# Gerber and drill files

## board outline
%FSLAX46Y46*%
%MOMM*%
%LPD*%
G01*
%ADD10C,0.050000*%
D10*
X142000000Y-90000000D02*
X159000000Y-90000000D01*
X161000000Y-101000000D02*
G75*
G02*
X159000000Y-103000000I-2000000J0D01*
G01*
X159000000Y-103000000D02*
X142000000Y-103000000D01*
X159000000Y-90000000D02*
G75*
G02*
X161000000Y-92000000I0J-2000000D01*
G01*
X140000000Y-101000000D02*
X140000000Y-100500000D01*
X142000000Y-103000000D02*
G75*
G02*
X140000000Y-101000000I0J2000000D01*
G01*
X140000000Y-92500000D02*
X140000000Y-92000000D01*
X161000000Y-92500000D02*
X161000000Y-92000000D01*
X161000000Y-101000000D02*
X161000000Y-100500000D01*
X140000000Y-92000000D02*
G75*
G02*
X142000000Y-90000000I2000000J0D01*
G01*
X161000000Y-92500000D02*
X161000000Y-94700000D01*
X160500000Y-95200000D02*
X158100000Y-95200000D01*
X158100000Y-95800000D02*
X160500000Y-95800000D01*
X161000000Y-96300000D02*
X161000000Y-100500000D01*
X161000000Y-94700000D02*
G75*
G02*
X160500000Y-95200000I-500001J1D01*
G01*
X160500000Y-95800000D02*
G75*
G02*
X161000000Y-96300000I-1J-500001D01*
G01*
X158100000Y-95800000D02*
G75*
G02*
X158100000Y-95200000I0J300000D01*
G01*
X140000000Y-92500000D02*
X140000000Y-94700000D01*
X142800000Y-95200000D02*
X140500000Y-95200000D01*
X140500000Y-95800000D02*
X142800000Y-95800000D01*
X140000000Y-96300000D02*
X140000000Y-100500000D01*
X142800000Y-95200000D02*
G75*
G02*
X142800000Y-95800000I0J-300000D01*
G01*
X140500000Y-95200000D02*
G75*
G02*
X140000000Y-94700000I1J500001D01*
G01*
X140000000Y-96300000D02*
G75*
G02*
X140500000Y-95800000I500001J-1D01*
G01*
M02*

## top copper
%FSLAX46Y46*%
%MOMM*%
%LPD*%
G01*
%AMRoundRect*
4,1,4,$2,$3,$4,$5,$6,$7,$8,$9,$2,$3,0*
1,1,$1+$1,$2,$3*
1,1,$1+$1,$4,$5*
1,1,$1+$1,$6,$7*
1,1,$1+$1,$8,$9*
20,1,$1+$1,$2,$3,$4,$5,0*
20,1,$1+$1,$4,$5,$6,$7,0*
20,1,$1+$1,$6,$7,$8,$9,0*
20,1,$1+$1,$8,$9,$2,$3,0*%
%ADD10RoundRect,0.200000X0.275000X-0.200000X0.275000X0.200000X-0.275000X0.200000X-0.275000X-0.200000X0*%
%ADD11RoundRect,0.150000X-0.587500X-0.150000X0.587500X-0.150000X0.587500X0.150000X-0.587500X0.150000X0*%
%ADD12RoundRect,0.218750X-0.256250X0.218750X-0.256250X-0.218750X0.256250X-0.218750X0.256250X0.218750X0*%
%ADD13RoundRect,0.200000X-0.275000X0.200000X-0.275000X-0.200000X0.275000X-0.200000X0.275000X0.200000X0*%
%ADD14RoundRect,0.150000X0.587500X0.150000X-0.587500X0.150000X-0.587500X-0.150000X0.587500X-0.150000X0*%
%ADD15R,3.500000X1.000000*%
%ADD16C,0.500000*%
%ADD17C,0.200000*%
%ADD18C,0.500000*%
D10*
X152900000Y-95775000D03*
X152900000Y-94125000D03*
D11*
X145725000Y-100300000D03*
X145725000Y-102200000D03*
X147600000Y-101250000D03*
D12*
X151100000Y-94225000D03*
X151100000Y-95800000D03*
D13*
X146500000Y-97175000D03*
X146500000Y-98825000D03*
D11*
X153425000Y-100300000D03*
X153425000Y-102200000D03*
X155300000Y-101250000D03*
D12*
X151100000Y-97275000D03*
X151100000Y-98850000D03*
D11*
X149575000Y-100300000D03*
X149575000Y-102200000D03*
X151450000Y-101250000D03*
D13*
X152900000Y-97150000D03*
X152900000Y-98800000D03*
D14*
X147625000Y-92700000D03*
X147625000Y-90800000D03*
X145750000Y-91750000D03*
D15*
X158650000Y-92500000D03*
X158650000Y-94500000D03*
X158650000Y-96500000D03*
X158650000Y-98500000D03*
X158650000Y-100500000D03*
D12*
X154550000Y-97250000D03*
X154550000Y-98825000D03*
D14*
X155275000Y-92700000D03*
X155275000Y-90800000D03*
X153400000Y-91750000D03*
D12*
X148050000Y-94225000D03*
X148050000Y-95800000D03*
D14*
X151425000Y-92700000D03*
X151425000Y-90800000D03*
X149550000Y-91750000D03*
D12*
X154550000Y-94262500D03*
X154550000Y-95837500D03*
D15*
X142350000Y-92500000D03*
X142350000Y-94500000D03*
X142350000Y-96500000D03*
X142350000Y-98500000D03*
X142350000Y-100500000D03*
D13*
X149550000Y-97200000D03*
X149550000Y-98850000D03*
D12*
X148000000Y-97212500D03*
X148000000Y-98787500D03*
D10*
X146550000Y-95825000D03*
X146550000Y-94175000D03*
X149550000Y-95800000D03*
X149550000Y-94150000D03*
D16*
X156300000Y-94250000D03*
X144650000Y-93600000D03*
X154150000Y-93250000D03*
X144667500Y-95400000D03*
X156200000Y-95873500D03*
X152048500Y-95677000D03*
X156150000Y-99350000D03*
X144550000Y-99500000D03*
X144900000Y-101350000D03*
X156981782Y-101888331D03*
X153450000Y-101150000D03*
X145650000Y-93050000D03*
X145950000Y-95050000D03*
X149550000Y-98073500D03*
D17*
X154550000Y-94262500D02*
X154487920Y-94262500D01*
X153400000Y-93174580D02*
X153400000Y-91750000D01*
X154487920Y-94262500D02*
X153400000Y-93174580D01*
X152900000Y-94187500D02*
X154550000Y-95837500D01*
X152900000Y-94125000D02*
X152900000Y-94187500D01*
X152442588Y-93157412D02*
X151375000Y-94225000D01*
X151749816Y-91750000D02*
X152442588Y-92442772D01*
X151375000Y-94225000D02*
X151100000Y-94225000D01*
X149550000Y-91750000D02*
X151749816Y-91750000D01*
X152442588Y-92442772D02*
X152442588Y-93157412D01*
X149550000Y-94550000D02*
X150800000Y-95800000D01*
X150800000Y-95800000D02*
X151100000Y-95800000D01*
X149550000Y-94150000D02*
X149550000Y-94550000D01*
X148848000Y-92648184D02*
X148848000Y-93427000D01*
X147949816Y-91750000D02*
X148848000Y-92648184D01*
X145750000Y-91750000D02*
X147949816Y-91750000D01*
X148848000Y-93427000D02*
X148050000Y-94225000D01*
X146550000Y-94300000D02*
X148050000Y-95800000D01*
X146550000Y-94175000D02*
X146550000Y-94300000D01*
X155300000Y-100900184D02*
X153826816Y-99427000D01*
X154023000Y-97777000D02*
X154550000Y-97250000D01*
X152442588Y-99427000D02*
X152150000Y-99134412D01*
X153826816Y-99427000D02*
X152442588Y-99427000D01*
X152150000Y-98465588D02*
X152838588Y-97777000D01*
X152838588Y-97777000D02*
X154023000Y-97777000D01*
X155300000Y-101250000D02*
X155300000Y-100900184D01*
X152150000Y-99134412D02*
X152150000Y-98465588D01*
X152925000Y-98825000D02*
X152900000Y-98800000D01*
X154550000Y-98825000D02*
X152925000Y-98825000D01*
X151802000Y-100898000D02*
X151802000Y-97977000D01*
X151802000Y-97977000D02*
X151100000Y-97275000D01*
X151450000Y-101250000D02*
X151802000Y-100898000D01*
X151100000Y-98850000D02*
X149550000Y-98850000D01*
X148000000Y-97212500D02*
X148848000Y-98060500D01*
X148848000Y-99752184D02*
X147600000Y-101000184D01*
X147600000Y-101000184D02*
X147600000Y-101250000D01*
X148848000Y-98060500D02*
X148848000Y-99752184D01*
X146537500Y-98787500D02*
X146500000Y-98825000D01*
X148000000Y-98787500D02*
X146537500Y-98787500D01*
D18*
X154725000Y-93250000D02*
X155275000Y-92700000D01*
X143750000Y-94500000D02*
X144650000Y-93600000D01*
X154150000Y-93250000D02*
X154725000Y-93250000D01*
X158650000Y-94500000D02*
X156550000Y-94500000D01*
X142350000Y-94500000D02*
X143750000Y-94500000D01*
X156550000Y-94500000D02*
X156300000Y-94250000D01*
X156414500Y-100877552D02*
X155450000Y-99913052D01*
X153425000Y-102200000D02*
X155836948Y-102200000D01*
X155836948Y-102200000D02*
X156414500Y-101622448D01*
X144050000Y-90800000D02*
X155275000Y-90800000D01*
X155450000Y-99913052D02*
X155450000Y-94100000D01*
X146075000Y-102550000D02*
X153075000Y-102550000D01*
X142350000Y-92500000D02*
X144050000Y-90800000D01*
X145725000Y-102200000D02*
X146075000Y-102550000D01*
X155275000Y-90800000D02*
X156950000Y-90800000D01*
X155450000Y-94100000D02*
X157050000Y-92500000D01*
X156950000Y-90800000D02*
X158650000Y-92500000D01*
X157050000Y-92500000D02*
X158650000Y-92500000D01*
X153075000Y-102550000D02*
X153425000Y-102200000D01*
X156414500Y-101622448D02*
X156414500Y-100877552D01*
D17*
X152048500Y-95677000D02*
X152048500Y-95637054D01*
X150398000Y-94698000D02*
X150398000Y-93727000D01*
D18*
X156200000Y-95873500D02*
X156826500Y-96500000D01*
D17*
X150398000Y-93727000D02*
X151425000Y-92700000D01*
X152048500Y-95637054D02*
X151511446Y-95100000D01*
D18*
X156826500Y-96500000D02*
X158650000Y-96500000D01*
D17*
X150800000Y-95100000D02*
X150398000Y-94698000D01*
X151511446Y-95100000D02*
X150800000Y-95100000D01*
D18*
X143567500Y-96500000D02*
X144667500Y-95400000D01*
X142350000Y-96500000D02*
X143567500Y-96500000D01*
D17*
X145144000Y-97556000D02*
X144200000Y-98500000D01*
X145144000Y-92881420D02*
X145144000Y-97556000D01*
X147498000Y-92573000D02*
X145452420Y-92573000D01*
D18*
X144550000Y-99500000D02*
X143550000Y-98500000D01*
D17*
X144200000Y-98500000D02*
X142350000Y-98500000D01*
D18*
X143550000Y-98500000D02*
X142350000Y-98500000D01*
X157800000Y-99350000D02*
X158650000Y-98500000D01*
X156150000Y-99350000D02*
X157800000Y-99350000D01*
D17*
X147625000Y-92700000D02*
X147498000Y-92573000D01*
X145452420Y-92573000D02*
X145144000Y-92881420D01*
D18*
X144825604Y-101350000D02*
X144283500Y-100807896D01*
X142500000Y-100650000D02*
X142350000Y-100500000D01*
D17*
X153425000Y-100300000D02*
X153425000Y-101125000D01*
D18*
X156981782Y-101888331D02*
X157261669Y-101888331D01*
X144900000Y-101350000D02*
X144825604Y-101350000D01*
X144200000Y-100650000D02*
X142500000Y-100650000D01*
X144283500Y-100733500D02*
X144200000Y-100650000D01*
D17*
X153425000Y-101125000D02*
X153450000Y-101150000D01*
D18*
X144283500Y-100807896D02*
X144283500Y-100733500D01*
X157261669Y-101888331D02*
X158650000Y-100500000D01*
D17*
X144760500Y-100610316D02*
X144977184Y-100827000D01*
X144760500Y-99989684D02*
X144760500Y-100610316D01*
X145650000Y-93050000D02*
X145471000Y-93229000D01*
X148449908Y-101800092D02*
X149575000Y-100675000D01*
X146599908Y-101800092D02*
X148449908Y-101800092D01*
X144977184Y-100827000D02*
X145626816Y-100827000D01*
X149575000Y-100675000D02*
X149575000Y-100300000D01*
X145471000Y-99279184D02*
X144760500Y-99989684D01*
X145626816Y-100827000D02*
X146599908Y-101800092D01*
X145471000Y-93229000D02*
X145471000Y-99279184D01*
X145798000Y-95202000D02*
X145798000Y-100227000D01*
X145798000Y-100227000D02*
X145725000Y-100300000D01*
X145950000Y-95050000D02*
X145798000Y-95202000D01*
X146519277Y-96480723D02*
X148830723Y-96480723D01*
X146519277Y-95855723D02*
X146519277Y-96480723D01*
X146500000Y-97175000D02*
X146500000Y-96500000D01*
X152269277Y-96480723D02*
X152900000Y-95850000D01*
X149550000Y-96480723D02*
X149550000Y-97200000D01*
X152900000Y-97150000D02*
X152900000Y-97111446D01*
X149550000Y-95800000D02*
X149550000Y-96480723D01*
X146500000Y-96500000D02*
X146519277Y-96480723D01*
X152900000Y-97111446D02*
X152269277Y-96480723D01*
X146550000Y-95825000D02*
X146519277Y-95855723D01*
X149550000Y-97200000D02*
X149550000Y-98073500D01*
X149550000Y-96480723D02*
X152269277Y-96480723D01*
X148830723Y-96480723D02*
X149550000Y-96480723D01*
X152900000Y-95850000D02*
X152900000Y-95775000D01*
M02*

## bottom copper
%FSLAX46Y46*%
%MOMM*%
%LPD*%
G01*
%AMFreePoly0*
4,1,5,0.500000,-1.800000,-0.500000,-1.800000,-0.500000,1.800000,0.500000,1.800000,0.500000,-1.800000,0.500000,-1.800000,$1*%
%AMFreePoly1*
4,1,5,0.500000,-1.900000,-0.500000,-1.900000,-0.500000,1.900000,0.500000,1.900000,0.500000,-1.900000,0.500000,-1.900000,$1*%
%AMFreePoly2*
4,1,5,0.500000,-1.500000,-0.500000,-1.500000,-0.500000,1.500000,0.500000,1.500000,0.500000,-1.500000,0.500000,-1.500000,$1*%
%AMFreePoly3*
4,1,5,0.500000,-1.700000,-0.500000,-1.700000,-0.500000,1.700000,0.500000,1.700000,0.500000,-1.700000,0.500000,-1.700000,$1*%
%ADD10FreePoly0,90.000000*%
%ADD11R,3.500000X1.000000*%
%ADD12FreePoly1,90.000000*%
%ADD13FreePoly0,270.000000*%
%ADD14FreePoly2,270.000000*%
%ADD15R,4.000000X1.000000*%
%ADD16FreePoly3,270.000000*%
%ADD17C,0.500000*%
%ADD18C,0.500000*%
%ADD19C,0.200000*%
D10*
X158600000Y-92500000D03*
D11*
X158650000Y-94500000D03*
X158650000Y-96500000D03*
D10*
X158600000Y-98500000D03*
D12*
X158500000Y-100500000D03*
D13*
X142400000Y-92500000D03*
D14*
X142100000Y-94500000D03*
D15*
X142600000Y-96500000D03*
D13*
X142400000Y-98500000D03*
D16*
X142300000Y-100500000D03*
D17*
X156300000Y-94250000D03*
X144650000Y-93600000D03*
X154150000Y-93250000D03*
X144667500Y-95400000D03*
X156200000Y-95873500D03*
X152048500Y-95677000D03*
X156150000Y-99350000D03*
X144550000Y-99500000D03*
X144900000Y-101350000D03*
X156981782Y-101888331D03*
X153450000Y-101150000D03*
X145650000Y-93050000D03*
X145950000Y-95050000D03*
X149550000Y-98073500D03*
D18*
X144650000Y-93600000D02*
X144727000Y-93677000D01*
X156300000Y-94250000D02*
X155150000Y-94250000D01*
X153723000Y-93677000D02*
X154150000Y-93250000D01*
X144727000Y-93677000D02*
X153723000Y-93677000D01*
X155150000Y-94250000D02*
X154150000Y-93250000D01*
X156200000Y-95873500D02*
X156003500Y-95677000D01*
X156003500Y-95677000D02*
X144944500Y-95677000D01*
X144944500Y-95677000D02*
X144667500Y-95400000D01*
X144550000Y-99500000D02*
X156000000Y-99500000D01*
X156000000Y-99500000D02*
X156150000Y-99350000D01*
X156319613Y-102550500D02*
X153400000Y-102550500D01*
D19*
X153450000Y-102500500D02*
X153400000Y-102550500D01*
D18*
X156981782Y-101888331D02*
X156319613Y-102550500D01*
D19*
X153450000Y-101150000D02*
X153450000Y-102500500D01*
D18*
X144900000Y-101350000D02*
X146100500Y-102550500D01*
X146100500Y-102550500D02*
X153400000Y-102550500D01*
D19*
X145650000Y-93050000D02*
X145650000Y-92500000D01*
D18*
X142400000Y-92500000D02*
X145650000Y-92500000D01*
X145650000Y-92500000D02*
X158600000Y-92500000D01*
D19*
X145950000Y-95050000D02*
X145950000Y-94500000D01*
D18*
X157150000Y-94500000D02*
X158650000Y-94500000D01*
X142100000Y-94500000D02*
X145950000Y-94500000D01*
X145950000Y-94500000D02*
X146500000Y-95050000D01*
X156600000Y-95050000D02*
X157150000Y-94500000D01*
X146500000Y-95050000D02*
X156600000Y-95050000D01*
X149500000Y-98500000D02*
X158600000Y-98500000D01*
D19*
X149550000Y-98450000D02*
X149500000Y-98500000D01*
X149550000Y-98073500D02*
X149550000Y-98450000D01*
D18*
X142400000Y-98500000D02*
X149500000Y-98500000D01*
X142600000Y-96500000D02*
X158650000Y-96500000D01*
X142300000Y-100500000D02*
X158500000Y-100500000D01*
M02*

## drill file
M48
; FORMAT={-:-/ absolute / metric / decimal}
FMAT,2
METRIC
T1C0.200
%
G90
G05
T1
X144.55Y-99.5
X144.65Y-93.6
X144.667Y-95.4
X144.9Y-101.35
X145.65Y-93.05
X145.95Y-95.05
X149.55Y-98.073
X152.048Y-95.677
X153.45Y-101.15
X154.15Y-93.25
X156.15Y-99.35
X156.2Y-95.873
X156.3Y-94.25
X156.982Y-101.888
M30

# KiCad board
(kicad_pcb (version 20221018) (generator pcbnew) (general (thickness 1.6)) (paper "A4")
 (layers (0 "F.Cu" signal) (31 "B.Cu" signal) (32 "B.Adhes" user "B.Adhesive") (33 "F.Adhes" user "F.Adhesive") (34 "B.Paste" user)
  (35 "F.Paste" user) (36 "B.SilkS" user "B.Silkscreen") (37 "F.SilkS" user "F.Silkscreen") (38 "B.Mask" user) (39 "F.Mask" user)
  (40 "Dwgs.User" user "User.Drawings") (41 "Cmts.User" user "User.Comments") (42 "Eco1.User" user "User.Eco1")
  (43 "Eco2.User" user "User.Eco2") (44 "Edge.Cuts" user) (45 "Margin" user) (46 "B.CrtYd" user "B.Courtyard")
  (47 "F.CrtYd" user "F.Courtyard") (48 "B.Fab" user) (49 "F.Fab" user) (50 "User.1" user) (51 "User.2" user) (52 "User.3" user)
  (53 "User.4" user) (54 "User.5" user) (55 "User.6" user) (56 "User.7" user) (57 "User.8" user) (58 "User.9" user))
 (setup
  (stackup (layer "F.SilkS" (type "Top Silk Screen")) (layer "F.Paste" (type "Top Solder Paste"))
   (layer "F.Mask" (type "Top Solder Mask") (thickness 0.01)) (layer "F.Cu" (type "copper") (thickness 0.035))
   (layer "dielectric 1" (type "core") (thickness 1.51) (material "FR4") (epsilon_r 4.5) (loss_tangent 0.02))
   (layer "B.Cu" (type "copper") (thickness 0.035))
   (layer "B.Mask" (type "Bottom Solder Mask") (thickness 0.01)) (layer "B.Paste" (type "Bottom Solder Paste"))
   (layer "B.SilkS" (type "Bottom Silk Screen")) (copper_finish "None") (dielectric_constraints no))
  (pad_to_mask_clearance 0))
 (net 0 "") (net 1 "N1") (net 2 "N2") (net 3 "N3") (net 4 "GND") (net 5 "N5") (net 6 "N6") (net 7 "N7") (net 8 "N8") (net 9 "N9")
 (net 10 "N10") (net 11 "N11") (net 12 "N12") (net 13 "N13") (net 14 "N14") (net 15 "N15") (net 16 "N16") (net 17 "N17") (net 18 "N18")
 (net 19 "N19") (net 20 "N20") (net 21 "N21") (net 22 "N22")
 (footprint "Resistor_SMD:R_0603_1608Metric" (layer "F.Cu") (at 152.9 94.95 90)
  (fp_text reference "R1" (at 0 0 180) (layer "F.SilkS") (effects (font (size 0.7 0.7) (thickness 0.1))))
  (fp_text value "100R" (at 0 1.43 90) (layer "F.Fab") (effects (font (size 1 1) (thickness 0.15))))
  (pad "1" smd roundrect (at -0.825 0 90) (size 0.8 0.95) (layers "F.Cu" "F.Paste" "F.Mask") (roundrect_rratio 0.25) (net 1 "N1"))
  (pad "2" smd roundrect (at 0.825 0 90) (size 0.8 0.95) (layers "F.Cu" "F.Paste" "F.Mask") (roundrect_rratio 0.25) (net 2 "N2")))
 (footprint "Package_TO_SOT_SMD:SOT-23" (layer "F.Cu") (at 146.6625 101.25)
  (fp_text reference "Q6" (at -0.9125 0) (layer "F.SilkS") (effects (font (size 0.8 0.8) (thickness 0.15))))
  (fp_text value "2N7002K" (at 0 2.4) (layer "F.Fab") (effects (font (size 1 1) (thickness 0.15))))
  (pad "1" smd roundrect (at -0.9375 -0.95) (size 1.475 0.6) (layers "F.Cu" "F.Paste" "F.Mask") (roundrect_rratio 0.25) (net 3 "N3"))
  (pad "2" smd roundrect (at -0.9375 0.95) (size 1.475 0.6) (layers "F.Cu" "F.Paste" "F.Mask") (roundrect_rratio 0.25) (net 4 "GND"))
  (pad "3" smd roundrect (at 0.9375 0) (size 1.475 0.6) (layers "F.Cu" "F.Paste" "F.Mask") (roundrect_rratio 0.25) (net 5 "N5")))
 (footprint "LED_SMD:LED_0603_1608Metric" (layer "F.Cu") (at 151.1 95.0125 -90)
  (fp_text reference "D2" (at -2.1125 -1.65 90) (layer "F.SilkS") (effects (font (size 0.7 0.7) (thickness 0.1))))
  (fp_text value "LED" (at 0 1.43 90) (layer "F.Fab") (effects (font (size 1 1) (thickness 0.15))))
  (pad "1" smd roundrect (at -0.7875 0 270) (size 0.875 0.95) (layers "F.Cu" "F.Paste" "F.Mask") (roundrect_rratio 0.25) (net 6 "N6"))
  (pad "2" smd roundrect (at 0.7875 0 270) (size 0.875 0.95) (layers "F.Cu" "F.Paste" "F.Mask") (roundrect_rratio 0.25) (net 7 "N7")))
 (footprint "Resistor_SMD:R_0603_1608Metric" (layer "F.Cu") (at 146.5 98 -90)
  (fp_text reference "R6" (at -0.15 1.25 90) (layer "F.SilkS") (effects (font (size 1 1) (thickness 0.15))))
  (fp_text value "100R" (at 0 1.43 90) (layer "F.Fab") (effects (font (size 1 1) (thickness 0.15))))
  (pad "1" smd roundrect (at -0.825 0 270) (size 0.8 0.95) (layers "F.Cu" "F.Paste" "F.Mask") (roundrect_rratio 0.25) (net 1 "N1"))
  (pad "2" smd roundrect (at 0.825 0 270) (size 0.8 0.95) (layers "F.Cu" "F.Paste" "F.Mask") (roundrect_rratio 0.25) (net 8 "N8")))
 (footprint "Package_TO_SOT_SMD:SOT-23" (layer "F.Cu") (at 154.3625 101.25)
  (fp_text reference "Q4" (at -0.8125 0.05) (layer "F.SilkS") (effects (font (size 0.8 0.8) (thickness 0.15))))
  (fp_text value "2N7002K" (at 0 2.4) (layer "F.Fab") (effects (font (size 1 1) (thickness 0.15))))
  (pad "1" smd roundrect (at -0.9375 -0.95) (size 1.475 0.6) (layers "F.Cu" "F.Paste" "F.Mask") (roundrect_rratio 0.25) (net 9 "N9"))
  (pad "2" smd roundrect (at -0.9375 0.95) (size 1.475 0.6) (layers "F.Cu" "F.Paste" "F.Mask") (roundrect_rratio 0.25) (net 4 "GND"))
  (pad "3" smd roundrect (at 0.9375 0) (size 1.475 0.6) (layers "F.Cu" "F.Paste" "F.Mask") (roundrect_rratio 0.25) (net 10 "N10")))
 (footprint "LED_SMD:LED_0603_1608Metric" (layer "F.Cu") (at 151.1 98.0625 -90)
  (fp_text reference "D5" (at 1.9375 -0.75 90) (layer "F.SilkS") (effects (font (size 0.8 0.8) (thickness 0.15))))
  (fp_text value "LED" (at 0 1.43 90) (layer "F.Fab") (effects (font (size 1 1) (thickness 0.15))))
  (pad "1" smd roundrect (at -0.7875 0 270) (size 0.875 0.95) (layers "F.Cu" "F.Paste" "F.Mask") (roundrect_rratio 0.25) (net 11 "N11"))
  (pad "2" smd roundrect (at 0.7875 0 270) (size 0.875 0.95) (layers "F.Cu" "F.Paste" "F.Mask") (roundrect_rratio 0.25) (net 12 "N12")))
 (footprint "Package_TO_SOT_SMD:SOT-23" (layer "F.Cu") (at 150.5125 101.25)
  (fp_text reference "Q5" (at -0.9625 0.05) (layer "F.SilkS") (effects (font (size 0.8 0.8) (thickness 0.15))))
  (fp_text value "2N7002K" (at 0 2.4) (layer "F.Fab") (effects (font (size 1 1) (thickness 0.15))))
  (pad "1" smd roundrect (at -0.9375 -0.95) (size 1.475 0.6) (layers "F.Cu" "F.Paste" "F.Mask") (roundrect_rratio 0.25) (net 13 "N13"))
  (pad "2" smd roundrect (at -0.9375 0.95) (size 1.475 0.6) (layers "F.Cu" "F.Paste" "F.Mask") (roundrect_rratio 0.25) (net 4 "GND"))
  (pad "3" smd roundrect (at 0.9375 0) (size 1.475 0.6) (layers "F.Cu" "F.Paste" "F.Mask") (roundrect_rratio 0.25) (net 11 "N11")))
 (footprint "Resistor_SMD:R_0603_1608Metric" (layer "F.Cu") (at 152.9 97.975 -90)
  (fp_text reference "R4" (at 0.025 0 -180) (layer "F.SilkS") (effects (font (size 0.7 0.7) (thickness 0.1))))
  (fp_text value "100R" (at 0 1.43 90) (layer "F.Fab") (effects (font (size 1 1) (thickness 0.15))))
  (pad "1" smd roundrect (at -0.825 0 270) (size 0.8 0.95) (layers "F.Cu" "F.Paste" "F.Mask") (roundrect_rratio 0.25) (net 1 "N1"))
  (pad "2" smd roundrect (at 0.825 0 270) (size 0.8 0.95) (layers "F.Cu" "F.Paste" "F.Mask") (roundrect_rratio 0.25) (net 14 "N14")))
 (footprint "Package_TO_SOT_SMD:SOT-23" (layer "F.Cu") (at 146.6875 91.75 180)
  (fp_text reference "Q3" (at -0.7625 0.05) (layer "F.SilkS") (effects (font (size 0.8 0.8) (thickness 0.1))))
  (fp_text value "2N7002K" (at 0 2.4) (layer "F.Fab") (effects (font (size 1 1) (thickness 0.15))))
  (pad "1" smd roundrect (at -0.9375 -0.95 180) (size 1.475 0.6) (layers "F.Cu" "F.Paste" "F.Mask") (roundrect_rratio 0.25) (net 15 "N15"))
  (pad "2" smd roundrect (at -0.9375 0.95 180) (size 1.475 0.6) (layers "F.Cu" "F.Paste" "F.Mask") (roundrect_rratio 0.25) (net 4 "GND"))
  (pad "3" smd roundrect (at 0.9375 0 180) (size 1.475 0.6) (layers "F.Cu" "F.Paste" "F.Mask") (roundrect_rratio 0.25) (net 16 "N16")))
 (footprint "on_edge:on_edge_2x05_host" (layer "F.Cu") (at 161 96.5 -90)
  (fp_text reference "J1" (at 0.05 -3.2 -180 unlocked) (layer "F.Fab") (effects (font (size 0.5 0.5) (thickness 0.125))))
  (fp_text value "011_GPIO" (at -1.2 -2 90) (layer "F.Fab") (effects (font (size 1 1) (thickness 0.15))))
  (fp_line (start -4 0) (end -1.8 0) (stroke (width 0.05) (type solid)) (layer "Edge.Cuts"))
  (fp_line (start -1.3 0.5) (end -1.3 2.9) (stroke (width 0.05) (type solid)) (layer "Edge.Cuts"))
  (fp_line (start -0.7 2.9) (end -0.7 0.5) (stroke (width 0.05) (type solid)) (layer "Edge.Cuts"))
  (fp_line (start -0.2 0) (end 4 0) (stroke (width 0.05) (type solid)) (layer "Edge.Cuts"))
  (fp_arc (start -1.8 0) (mid -1.446447 0.146447) (end -1.3 0.5) (stroke (width 0.05) (type solid)) (layer "Edge.Cuts"))
  (fp_arc (start -0.7 0.5) (mid -0.553553 0.146447) (end -0.2 0) (stroke (width 0.05) (type solid)) (layer "Edge.Cuts"))
  (fp_arc (start -0.7 2.9) (mid -1 3.2) (end -1.3 2.9) (stroke (width 0.05) (type solid)) (layer "Edge.Cuts"))
  (pad "1" smd rect (at -4 2.35 270) (size 1 3.5) (layers "F.Cu" "F.Mask") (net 4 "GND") (zone_connect 0))
  (pad "2" smd rect (at -2 2.35 270) (size 1 3.5) (layers "F.Cu" "F.Mask") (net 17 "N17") (zone_connect 0))
  (pad "3" smd rect (at 0 2.35 270) (size 1 3.5) (layers "F.Cu" "F.Mask") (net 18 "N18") (zone_connect 0))
  (pad "4" smd rect (at 2 2.35 270) (size 1 3.5) (layers "F.Cu" "F.Mask") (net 15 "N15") (zone_connect 0))
  (pad "5" smd rect (at 4 2.35 270) (size 1 3.5) (layers "F.Cu" "F.Mask") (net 9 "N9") (zone_connect 0))
  (pad "6" smd custom (at -4 2.4 90) (size 1 3.6) (layers "B.Cu" "B.Mask") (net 13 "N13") (zone_connect 0)
   (options (clearance outline) (anchor rect)) (primitives))
  (pad "7" smd rect (at -2 2.35 90) (size 1 3.5) (layers "B.Cu" "B.Mask") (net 3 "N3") (zone_connect 0))
  (pad "8" smd rect (at 0 2.35 90) (size 1 3.5) (layers "B.Cu" "B.Mask") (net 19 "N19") (zone_connect 0))
  (pad "9" smd custom (at 2 2.4 90) (size 1 3.6) (layers "B.Cu" "B.Mask") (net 1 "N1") (zone_connect 0)
   (options (clearance outline) (anchor rect)) (primitives))
  (pad "10" smd custom (at 4 2.5 90) (size 1 3.8) (layers "B.Cu" "B.Mask") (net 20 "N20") (zone_connect 0)
   (options (clearance outline) (anchor rect)) (primitives))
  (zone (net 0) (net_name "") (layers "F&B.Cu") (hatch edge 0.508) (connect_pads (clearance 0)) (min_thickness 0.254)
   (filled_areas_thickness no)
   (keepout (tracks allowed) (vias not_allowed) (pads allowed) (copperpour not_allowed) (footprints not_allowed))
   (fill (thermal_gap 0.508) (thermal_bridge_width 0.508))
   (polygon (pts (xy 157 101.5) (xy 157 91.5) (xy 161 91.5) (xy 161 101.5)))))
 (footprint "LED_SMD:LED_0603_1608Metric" (layer "F.Cu") (at 154.55 98.0375 -90)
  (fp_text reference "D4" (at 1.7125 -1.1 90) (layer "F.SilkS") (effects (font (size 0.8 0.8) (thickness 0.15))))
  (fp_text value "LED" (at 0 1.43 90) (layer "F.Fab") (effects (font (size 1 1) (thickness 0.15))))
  (pad "1" smd roundrect (at -0.7875 0 270) (size 0.875 0.95) (layers "F.Cu" "F.Paste" "F.Mask") (roundrect_rratio 0.25) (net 10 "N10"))
  (pad "2" smd roundrect (at 0.7875 0 270) (size 0.875 0.95) (layers "F.Cu" "F.Paste" "F.Mask") (roundrect_rratio 0.25) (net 14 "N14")))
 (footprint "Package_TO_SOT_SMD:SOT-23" (layer "F.Cu") (at 154.3375 91.75 180)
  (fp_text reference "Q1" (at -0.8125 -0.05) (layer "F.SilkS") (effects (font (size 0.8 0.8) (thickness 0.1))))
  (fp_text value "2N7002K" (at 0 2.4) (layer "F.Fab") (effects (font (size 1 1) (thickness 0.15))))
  (pad "1" smd roundrect (at -0.9375 -0.95 180) (size 1.475 0.6) (layers "F.Cu" "F.Paste" "F.Mask") (roundrect_rratio 0.25) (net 17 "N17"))
  (pad "2" smd roundrect (at -0.9375 0.95 180) (size 1.475 0.6) (layers "F.Cu" "F.Paste" "F.Mask") (roundrect_rratio 0.25) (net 4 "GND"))
  (pad "3" smd roundrect (at 0.9375 0 180) (size 1.475 0.6) (layers "F.Cu" "F.Paste" "F.Mask") (roundrect_rratio 0.25) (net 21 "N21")))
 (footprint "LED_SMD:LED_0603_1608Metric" (layer "F.Cu") (at 148.05 95.0125 -90)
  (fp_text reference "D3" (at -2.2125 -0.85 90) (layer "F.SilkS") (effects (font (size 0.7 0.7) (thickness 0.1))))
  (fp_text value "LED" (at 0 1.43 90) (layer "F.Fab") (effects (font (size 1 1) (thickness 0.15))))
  (pad "1" smd roundrect (at -0.7875 0 270) (size 0.875 0.95) (layers "F.Cu" "F.Paste" "F.Mask") (roundrect_rratio 0.25) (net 16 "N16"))
  (pad "2" smd roundrect (at 0.7875 0 270) (size 0.875 0.95) (layers "F.Cu" "F.Paste" "F.Mask") (roundrect_rratio 0.25) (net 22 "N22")))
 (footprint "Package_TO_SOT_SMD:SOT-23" (layer "F.Cu") (at 150.4875 91.75 180)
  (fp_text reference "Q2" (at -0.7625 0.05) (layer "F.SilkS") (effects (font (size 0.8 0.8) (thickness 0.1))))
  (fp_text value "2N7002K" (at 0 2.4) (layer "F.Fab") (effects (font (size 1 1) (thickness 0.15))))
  (pad "1" smd roundrect (at -0.9375 -0.95 180) (size 1.475 0.6) (layers "F.Cu" "F.Paste" "F.Mask") (roundrect_rratio 0.25) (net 18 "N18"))
  (pad "2" smd roundrect (at -0.9375 0.95 180) (size 1.475 0.6) (layers "F.Cu" "F.Paste" "F.Mask") (roundrect_rratio 0.25) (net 4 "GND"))
  (pad "3" smd roundrect (at 0.9375 0 180) (size 1.475 0.6) (layers "F.Cu" "F.Paste" "F.Mask") (roundrect_rratio 0.25) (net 6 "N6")))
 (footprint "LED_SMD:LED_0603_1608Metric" (layer "F.Cu") (at 154.55 95.05 -90)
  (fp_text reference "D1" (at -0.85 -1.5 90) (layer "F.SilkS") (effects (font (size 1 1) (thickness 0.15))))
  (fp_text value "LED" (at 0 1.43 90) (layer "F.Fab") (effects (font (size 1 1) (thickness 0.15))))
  (pad "1" smd roundrect (at -0.7875 0 270) (size 0.875 0.95) (layers "F.Cu" "F.Paste" "F.Mask") (roundrect_rratio 0.25) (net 21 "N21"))
  (pad "2" smd roundrect (at 0.7875 0 270) (size 0.875 0.95) (layers "F.Cu" "F.Paste" "F.Mask") (roundrect_rratio 0.25) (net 2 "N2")))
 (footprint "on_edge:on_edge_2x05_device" (layer "F.Cu") (at 140 96.5 -90)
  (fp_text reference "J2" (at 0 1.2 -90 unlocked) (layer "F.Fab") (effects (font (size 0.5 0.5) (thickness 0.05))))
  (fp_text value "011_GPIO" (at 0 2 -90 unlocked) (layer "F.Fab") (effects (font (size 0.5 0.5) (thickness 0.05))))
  (fp_line (start -4 0) (end -1.8 0) (stroke (width 0.05) (type solid)) (layer "Edge.Cuts"))
  (fp_line (start -1.3 -2.8) (end -1.3 -0.5) (stroke (width 0.05) (type solid)) (layer "Edge.Cuts"))
  (fp_line (start -0.7 -0.5) (end -0.7 -2.8) (stroke (width 0.05) (type solid)) (layer "Edge.Cuts"))
  (fp_line (start -0.2 0) (end 4 0) (stroke (width 0.05) (type solid)) (layer "Edge.Cuts"))
  (fp_arc (start -1.3 -2.8) (mid -1 -3.1) (end -0.7 -2.8) (stroke (width 0.05) (type solid)) (layer "Edge.Cuts"))
  (fp_arc (start -1.3 -0.5) (mid -1.446447 -0.146447) (end -1.8 0) (stroke (width 0.05) (type solid)) (layer "Edge.Cuts"))
  (fp_arc (start -0.2 0) (mid -0.553553 -0.146447) (end -0.7 -0.5) (stroke (width 0.05) (type solid)) (layer "Edge.Cuts"))
  (pad "1" smd rect (at -4 -2.35 90) (size 1 3.5) (layers "F.Cu" "F.Mask") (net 4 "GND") (zone_connect 0))
  (pad "2" smd rect (at -2 -2.35 270) (size 1 3.5) (layers "F.Cu" "F.Mask") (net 17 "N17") (zone_connect 0))
  (pad "3" smd rect (at 0 -2.35 270) (size 1 3.5) (layers "F.Cu" "F.Mask") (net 18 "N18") (zone_connect 0))
  (pad "4" smd rect (at 2 -2.35 90) (size 1 3.5) (layers "F.Cu" "F.Mask") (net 15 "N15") (zone_connect 0))
  (pad "5" smd rect (at 4 -2.35 90) (size 1 3.5) (layers "F.Cu" "F.Mask") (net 9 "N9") (zone_connect 0))
  (pad "6" smd custom (at -4 -2.4 270) (size 1 3.6) (layers "B.Cu" "B.Mask") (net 13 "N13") (zone_connect 0)
   (options (clearance outline) (anchor rect)) (primitives))
  (pad "7" smd custom (at -2 -2.1 270) (size 1 3) (layers "B.Cu" "B.Mask") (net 3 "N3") (zone_connect 0)
   (options (clearance outline) (anchor rect)) (primitives))
  (pad "8" smd rect (at 0 -2.6 270) (size 1 4) (layers "B.Cu" "B.Mask") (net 19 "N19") (zone_connect 0))
  (pad "9" smd custom (at 2 -2.4 270) (size 1 3.6) (layers "B.Cu" "B.Mask") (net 1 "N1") (zone_connect 0)
   (options (clearance outline) (anchor rect)) (primitives))
  (pad "10" smd custom (at 4 -2.3 270) (size 1 3.4) (layers "B.Cu" "B.Mask") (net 20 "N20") (zone_connect 0)
   (options (clearance outline) (anchor rect)) (primitives))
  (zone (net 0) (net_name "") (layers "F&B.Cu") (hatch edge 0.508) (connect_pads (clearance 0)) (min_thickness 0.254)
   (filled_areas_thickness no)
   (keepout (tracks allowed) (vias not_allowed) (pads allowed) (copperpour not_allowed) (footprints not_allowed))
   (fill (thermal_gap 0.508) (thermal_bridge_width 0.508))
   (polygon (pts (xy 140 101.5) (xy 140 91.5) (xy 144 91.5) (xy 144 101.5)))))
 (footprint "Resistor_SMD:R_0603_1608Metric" (layer "F.Cu") (at 149.55 98.025 -90)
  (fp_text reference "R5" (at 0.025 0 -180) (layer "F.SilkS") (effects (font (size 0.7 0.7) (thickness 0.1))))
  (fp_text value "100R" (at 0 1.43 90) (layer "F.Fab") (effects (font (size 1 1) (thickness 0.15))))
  (pad "1" smd roundrect (at -0.825 0 270) (size 0.8 0.95) (layers "F.Cu" "F.Paste" "F.Mask") (roundrect_rratio 0.25) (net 1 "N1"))
  (pad "2" smd roundrect (at 0.825 0 270) (size 0.8 0.95) (layers "F.Cu" "F.Paste" "F.Mask") (roundrect_rratio 0.25) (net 12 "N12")))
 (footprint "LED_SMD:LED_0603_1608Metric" (layer "F.Cu") (at 148 98 -90)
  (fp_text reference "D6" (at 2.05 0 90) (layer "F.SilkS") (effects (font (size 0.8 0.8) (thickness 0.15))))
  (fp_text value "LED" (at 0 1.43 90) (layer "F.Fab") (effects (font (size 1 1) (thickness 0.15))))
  (pad "1" smd roundrect (at -0.7875 0 270) (size 0.875 0.95) (layers "F.Cu" "F.Paste" "F.Mask") (roundrect_rratio 0.25) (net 5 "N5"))
  (pad "2" smd roundrect (at 0.7875 0 270) (size 0.875 0.95) (layers "F.Cu" "F.Paste" "F.Mask") (roundrect_rratio 0.25) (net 8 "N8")))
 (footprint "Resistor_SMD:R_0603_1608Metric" (layer "F.Cu") (at 146.55 95 90)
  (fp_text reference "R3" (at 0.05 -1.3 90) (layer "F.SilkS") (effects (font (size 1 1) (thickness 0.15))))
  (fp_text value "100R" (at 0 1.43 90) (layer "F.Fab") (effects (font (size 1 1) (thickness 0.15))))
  (pad "1" smd roundrect (at -0.825 0 90) (size 0.8 0.95) (layers "F.Cu" "F.Paste" "F.Mask") (roundrect_rratio 0.25) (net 1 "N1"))
  (pad "2" smd roundrect (at 0.825 0 90) (size 0.8 0.95) (layers "F.Cu" "F.Paste" "F.Mask") (roundrect_rratio 0.25) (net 22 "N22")))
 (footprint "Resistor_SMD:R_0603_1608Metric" (layer "F.Cu") (at 149.55 94.975 90)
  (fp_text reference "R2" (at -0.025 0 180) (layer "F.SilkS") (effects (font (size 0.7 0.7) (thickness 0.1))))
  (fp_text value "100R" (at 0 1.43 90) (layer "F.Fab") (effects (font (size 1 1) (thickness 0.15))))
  (pad "1" smd roundrect (at -0.825 0 90) (size 0.8 0.95) (layers "F.Cu" "F.Paste" "F.Mask") (roundrect_rratio 0.25) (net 1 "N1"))
  (pad "2" smd roundrect (at 0.825 0 90) (size 0.8 0.95) (layers "F.Cu" "F.Paste" "F.Mask") (roundrect_rratio 0.25) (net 7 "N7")))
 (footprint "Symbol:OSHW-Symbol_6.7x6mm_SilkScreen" (layer "B.Cu") (at 150.65 99.25 180)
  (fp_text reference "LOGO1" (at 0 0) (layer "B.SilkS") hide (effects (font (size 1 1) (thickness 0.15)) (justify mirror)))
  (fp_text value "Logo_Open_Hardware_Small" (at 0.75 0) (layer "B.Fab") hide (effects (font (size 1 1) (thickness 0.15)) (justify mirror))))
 (gr_line (start 142 90) (end 159 90) (stroke (width 0.05) (type solid)) (layer "Edge.Cuts"))
 (gr_arc (start 161 101) (mid 160.414214 102.414214) (end 159 103) (stroke (width 0.05) (type solid)) (layer "Edge.Cuts"))
 (gr_line (start 159 103) (end 142 103) (stroke (width 0.05) (type solid)) (layer "Edge.Cuts"))
 (gr_arc (start 159 90) (mid 160.414214 90.585786) (end 161 92) (stroke (width 0.05) (type solid)) (layer "Edge.Cuts"))
 (gr_line (start 140 101) (end 140 100.5) (stroke (width 0.05) (type solid)) (layer "Edge.Cuts"))
 (gr_arc (start 142 103) (mid 140.585786 102.414214) (end 140 101) (stroke (width 0.05) (type solid)) (layer "Edge.Cuts"))
 (gr_line (start 140 92.5) (end 140 92) (stroke (width 0.05) (type solid)) (layer "Edge.Cuts"))
 (gr_line (start 161 92.5) (end 161 92) (stroke (width 0.05) (type solid)) (layer "Edge.Cuts"))
 (gr_line (start 161 101) (end 161 100.5) (stroke (width 0.05) (type solid)) (layer "Edge.Cuts"))
 (gr_arc (start 140 92) (mid 140.585786 90.585786) (end 142 90) (stroke (width 0.05) (type solid)) (layer "Edge.Cuts"))
 (segment (start 154.55 94.2625) (end 154.48792 94.2625) (width 0.2) (layer "F.Cu") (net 21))
 (segment (start 153.4 93.17458) (end 153.4 91.75) (width 0.2) (layer "F.Cu") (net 21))
 (segment (start 154.48792 94.2625) (end 153.4 93.17458) (width 0.2) (layer "F.Cu") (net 21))
 (segment (start 152.9 94.1875) (end 154.55 95.8375) (width 0.2) (layer "F.Cu") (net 2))
 (segment (start 152.9 94.125) (end 152.9 94.1875) (width 0.2) (layer "F.Cu") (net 2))
 (segment (start 152.442588 93.157412) (end 151.375 94.225) (width 0.2) (layer "F.Cu") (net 6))
 (segment (start 151.749816 91.75) (end 152.442588 92.442772) (width 0.2) (layer "F.Cu") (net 6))
 (segment (start 151.375 94.225) (end 151.1 94.225) (width 0.2) (layer "F.Cu") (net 6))
 (segment (start 149.55 91.75) (end 151.749816 91.75) (width 0.2) (layer "F.Cu") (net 6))
 (segment (start 152.442588 92.442772) (end 152.442588 93.157412) (width 0.2) (layer "F.Cu") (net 6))
 (segment (start 149.55 94.55) (end 150.8 95.8) (width 0.2) (layer "F.Cu") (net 7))
 (segment (start 150.8 95.8) (end 151.1 95.8) (width 0.2) (layer "F.Cu") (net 7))
 (segment (start 149.55 94.15) (end 149.55 94.55) (width 0.2) (layer "F.Cu") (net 7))
 (segment (start 148.848 92.648184) (end 148.848 93.427) (width 0.2) (layer "F.Cu") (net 16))
 (segment (start 147.949816 91.75) (end 148.848 92.648184) (width 0.2) (layer "F.Cu") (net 16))
 (segment (start 145.75 91.75) (end 147.949816 91.75) (width 0.2) (layer "F.Cu") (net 16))
 (segment (start 148.848 93.427) (end 148.05 94.225) (width 0.2) (layer "F.Cu") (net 16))
 (segment (start 146.55 94.3) (end 148.05 95.8) (width 0.2) (layer "F.Cu") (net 22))
 (segment (start 146.55 94.175) (end 146.55 94.3) (width 0.2) (layer "F.Cu") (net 22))
 (segment (start 155.3 100.900184) (end 153.826816 99.427) (width 0.2) (layer "F.Cu") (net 10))
 (segment (start 154.023 97.777) (end 154.55 97.25) (width 0.2) (layer "F.Cu") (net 10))
 (segment (start 152.442588 99.427) (end 152.15 99.134412) (width 0.2) (layer "F.Cu") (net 10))
 (segment (start 153.826816 99.427) (end 152.442588 99.427) (width 0.2) (layer "F.Cu") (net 10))
 (segment (start 152.15 98.465588) (end 152.838588 97.777) (width 0.2) (layer "F.Cu") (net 10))
 (segment (start 152.838588 97.777) (end 154.023 97.777) (width 0.2) (layer "F.Cu") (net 10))
 (segment (start 155.3 101.25) (end 155.3 100.900184) (width 0.2) (layer "F.Cu") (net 10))
 (segment (start 152.15 99.134412) (end 152.15 98.465588) (width 0.2) (layer "F.Cu") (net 10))
 (segment (start 152.925 98.825) (end 152.9 98.8) (width 0.2) (layer "F.Cu") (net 14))
 (segment (start 154.55 98.825) (end 152.925 98.825) (width 0.2) (layer "F.Cu") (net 14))
 (segment (start 151.802 100.898) (end 151.802 97.977) (width 0.2) (layer "F.Cu") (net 11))
 (segment (start 151.802 97.977) (end 151.1 97.275) (width 0.2) (layer "F.Cu") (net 11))
 (segment (start 151.45 101.25) (end 151.802 100.898) (width 0.2) (layer "F.Cu") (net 11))
 (segment (start 151.1 98.85) (end 149.55 98.85) (width 0.2) (layer "F.Cu") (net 12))
 (segment (start 148 97.2125) (end 148.848 98.0605) (width 0.2) (layer "F.Cu") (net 5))
 (segment (start 148.848 99.752184) (end 147.6 101.000184) (width 0.2) (layer "F.Cu") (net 5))
 (segment (start 147.6 101.000184) (end 147.6 101.25) (width 0.2) (layer "F.Cu") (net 5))
 (segment (start 148.848 98.0605) (end 148.848 99.752184) (width 0.2) (layer "F.Cu") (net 5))
 (segment (start 146.5375 98.7875) (end 146.5 98.825) (width 0.2) (layer "F.Cu") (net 8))
 (segment (start 148 98.7875) (end 146.5375 98.7875) (width 0.2) (layer "F.Cu") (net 8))
 (segment (start 154.725 93.25) (end 155.275 92.7) (width 0.5) (layer "F.Cu") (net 17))
 (segment (start 143.75 94.5) (end 144.65 93.6) (width 0.5) (layer "F.Cu") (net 17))
 (segment (start 154.15 93.25) (end 154.725 93.25) (width 0.5) (layer "F.Cu") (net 17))
 (segment (start 158.65 94.5) (end 156.55 94.5) (width 0.5) (layer "F.Cu") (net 17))
 (segment (start 142.35 94.5) (end 143.75 94.5) (width 0.5) (layer "F.Cu") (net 17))
 (segment (start 156.55 94.5) (end 156.3 94.25) (width 0.5) (layer "F.Cu") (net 17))
 (via (at 156.3 94.25) (size 0.5) (drill 0.2) (layers "F.Cu" "B.Cu") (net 17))
 (via (at 144.65 93.6) (size 0.5) (drill 0.2) (layers "F.Cu" "B.Cu") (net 17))
 (via (at 154.15 93.25) (size 0.5) (drill 0.2) (layers "F.Cu" "B.Cu") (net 17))
 (segment (start 144.65 93.6) (end 144.727 93.677) (width 0.5) (layer "B.Cu") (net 17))
 (segment (start 156.3 94.25) (end 155.15 94.25) (width 0.5) (layer "B.Cu") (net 17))
 (segment (start 153.723 93.677) (end 154.15 93.25) (width 0.5) (layer "B.Cu") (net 17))
 (segment (start 144.727 93.677) (end 153.723 93.677) (width 0.5) (layer "B.Cu") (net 17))
 (segment (start 155.15 94.25) (end 154.15 93.25) (width 0.5) (layer "B.Cu") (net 17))
 (segment (start 156.4145 100.877552) (end 155.45 99.913052) (width 0.5) (layer "F.Cu") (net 4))
 (segment (start 153.425 102.2) (end 155.836948 102.2) (width 0.5) (layer "F.Cu") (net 4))
 (segment (start 155.836948 102.2) (end 156.4145 101.622448) (width 0.5) (layer "F.Cu") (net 4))
 (segment (start 144.05 90.8) (end 155.275 90.8) (width 0.5) (layer "F.Cu") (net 4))
 (segment (start 155.45 99.913052) (end 155.45 94.1) (width 0.5) (layer "F.Cu") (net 4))
 (segment (start 146.075 102.55) (end 153.075 102.55) (width 0.5) (layer "F.Cu") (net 4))
 (segment (start 142.35 92.5) (end 144.05 90.8) (width 0.5) (layer "F.Cu") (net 4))
 (segment (start 145.725 102.2) (end 146.075 102.55) (width 0.5) (layer "F.Cu") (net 4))
 (segment (start 155.275 90.8) (end 156.95 90.8) (width 0.5) (layer "F.Cu") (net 4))
 (segment (start 155.45 94.1) (end 157.05 92.5) (width 0.5) (layer "F.Cu") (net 4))
 (segment (start 156.95 90.8) (end 158.65 92.5) (width 0.5) (layer "F.Cu") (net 4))
 (segment (start 157.05 92.5) (end 158.65 92.5) (width 0.5) (layer "F.Cu") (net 4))
 (segment (start 153.075 102.55) (end 153.425 102.2) (width 0.5) (layer "F.Cu") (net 4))
 (segment (start 156.4145 101.622448) (end 156.4145 100.877552) (width 0.5) (layer "F.Cu") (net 4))
 (segment (start 152.0485 95.677) (end 152.0485 95.637054) (width 0.2) (layer "F.Cu") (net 18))
 (segment (start 150.398 94.698) (end 150.398 93.727) (width 0.2) (layer "F.Cu") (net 18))
 (segment (start 156.2 95.8735) (end 156.8265 96.5) (width 0.5) (layer "F.Cu") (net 18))
 (segment (start 150.398 93.727) (end 151.425 92.7) (width 0.2) (layer "F.Cu") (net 18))
 (segment (start 152.0485 95.637054) (end 151.511446 95.1) (width 0.2) (layer "F.Cu") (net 18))
 (segment (start 156.8265 96.5) (end 158.65 96.5) (width 0.5) (layer "F.Cu") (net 18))
 (segment (start 150.8 95.1) (end 150.398 94.698) (width 0.2) (layer "F.Cu") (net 18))
 (segment (start 151.511446 95.1) (end 150.8 95.1) (width 0.2) (layer "F.Cu") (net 18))
 (segment (start 143.5675 96.5) (end 144.6675 95.4) (width 0.5) (layer "F.Cu") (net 18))
 (segment (start 142.35 96.5) (end 143.5675 96.5) (width 0.5) (layer "F.Cu") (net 18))
 (via (at 144.6675 95.4) (size 0.5) (drill 0.2) (layers "F.Cu" "B.Cu") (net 18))
 (via (at 156.2 95.8735) (size 0.5) (drill 0.2) (layers "F.Cu" "B.Cu") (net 18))
 (via (at 152.0485 95.677) (size 0.5) (drill 0.2) (layers "F.Cu" "B.Cu") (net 18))
 (segment (start 156.2 95.8735) (end 156.0035 95.677) (width 0.5) (layer "B.Cu") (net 18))
 (segment (start 156.0035 95.677) (end 144.9445 95.677) (width 0.5) (layer "B.Cu") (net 18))
 (segment (start 144.9445 95.677) (end 144.6675 95.4) (width 0.5) (layer "B.Cu") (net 18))
 (segment (start 145.144 97.556) (end 144.2 98.5) (width 0.2) (layer "F.Cu") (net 15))
 (segment (start 145.144 92.88142) (end 145.144 97.556) (width 0.2) (layer "F.Cu") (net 15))
 (segment (start 147.498 92.573) (end 145.45242 92.573) (width 0.2) (layer "F.Cu") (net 15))
 (segment (start 144.55 99.5) (end 143.55 98.5) (width 0.5) (layer "F.Cu") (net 15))
 (segment (start 144.2 98.5) (end 142.35 98.5) (width 0.2) (layer "F.Cu") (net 15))
 (segment (start 143.55 98.5) (end 142.35 98.5) (width 0.5) (layer "F.Cu") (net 15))
 (segment (start 157.8 99.35) (end 158.65 98.5) (width 0.5) (layer "F.Cu") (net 15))
 (segment (start 156.15 99.35) (end 157.8 99.35) (width 0.5) (layer "F.Cu") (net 15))
 (segment (start 147.625 92.7) (end 147.498 92.573) (width 0.2) (layer "F.Cu") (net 15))
 (segment (start 145.45242 92.573) (end 145.144 92.88142) (width 0.2) (layer "F.Cu") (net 15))
 (via (at 156.15 99.35) (size 0.5) (drill 0.2) (layers "F.Cu" "B.Cu") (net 15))
 (via (at 144.55 99.5) (size 0.5) (drill 0.2) (layers "F.Cu" "B.Cu") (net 15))
 (segment (start 144.55 99.5) (end 156 99.5) (width 0.5) (layer "B.Cu") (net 15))
 (segment (start 156 99.5) (end 156.15 99.35) (width 0.5) (layer "B.Cu") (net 15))
 (segment (start 144.825604 101.35) (end 144.2835 100.807896) (width 0.5) (layer "F.Cu") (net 9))
 (segment (start 142.5 100.65) (end 142.35 100.5) (width 0.5) (layer "F.Cu") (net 9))
 (segment (start 153.425 100.3) (end 153.425 101.125) (width 0.2) (layer "F.Cu") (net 9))
 (segment (start 156.981782 101.888331) (end 157.261669 101.888331) (width 0.5) (layer "F.Cu") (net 9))
 (segment (start 144.9 101.35) (end 144.825604 101.35) (width 0.5) (layer "F.Cu") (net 9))
 (segment (start 144.2 100.65) (end 142.5 100.65) (width 0.5) (layer "F.Cu") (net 9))
 (segment (start 144.2835 100.7335) (end 144.2 100.65) (width 0.5) (layer "F.Cu") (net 9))
 (segment (start 153.425 101.125) (end 153.45 101.15) (width 0.2) (layer "F.Cu") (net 9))
 (segment (start 144.2835 100.807896) (end 144.2835 100.7335) (width 0.5) (layer "F.Cu") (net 9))
 (segment (start 157.261669 101.888331) (end 158.65 100.5) (width 0.5) (layer "F.Cu") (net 9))
 (via (at 144.9 101.35) (size 0.5) (drill 0.2) (layers "F.Cu" "B.Cu") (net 9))
 (via (at 156.981782 101.888331) (size 0.5) (drill 0.2) (layers "F.Cu" "B.Cu") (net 9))
 (via (at 153.45 101.15) (size 0.5) (drill 0.2) (layers "F.Cu" "B.Cu") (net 9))
 (segment (start 156.319613 102.5505) (end 153.4 102.5505) (width 0.5) (layer "B.Cu") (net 9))
 (segment (start 153.45 102.5005) (end 153.4 102.5505) (width 0.2) (layer "B.Cu") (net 9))
 (segment (start 156.981782 101.888331) (end 156.319613 102.5505) (width 0.5) (layer "B.Cu") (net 9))
 (segment (start 153.45 101.15) (end 153.45 102.5005) (width 0.2) (layer "B.Cu") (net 9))
 (segment (start 144.9 101.35) (end 146.1005 102.5505) (width 0.5) (layer "B.Cu") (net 9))
 (segment (start 146.1005 102.5505) (end 153.4 102.5505) (width 0.5) (layer "B.Cu") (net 9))
 (segment (start 144.7605 100.610316) (end 144.977184 100.827) (width 0.2) (layer "F.Cu") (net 13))
 (segment (start 144.7605 99.989684) (end 144.7605 100.610316) (width 0.2) (layer "F.Cu") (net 13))
 (segment (start 145.65 93.05) (end 145.471 93.229) (width 0.2) (layer "F.Cu") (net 13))
 (segment (start 148.449908 101.800092) (end 149.575 100.675) (width 0.2) (layer "F.Cu") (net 13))
 (segment (start 146.599908 101.800092) (end 148.449908 101.800092) (width 0.2) (layer "F.Cu") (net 13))
 (segment (start 144.977184 100.827) (end 145.626816 100.827) (width 0.2) (layer "F.Cu") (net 13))
 (segment (start 149.575 100.675) (end 149.575 100.3) (width 0.2) (layer "F.Cu") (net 13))
 (segment (start 145.471 99.279184) (end 144.7605 99.989684) (width 0.2) (layer "F.Cu") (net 13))
 (segment (start 145.626816 100.827) (end 146.599908 101.800092) (width 0.2) (layer "F.Cu") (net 13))
 (segment (start 145.471 93.229) (end 145.471 99.279184) (width 0.2) (layer "F.Cu") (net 13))
 (via (at 145.65 93.05) (size 0.5) (drill 0.2) (layers "F.Cu" "B.Cu") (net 13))
 (segment (start 145.65 93.05) (end 145.65 92.5) (width 0.2) (layer "B.Cu") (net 13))
 (segment (start 142.4 92.5) (end 145.65 92.5) (width 0.5) (layer "B.Cu") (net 13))
 (segment (start 145.65 92.5) (end 158.6 92.5) (width 0.5) (layer "B.Cu") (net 13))
 (segment (start 145.798 95.202) (end 145.798 100.227) (width 0.2) (layer "F.Cu") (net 3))
 (segment (start 145.798 100.227) (end 145.725 100.3) (width 0.2) (layer "F.Cu") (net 3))
 (segment (start 145.95 95.05) (end 145.798 95.202) (width 0.2) (layer "F.Cu") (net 3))
 (via (at 145.95 95.05) (size 0.5) (drill 0.2) (layers "F.Cu" "B.Cu") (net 3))
 (segment (start 145.95 95.05) (end 145.95 94.5) (width 0.2) (layer "B.Cu") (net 3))
 (segment (start 157.15 94.5) (end 158.65 94.5) (width 0.5) (layer "B.Cu") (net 3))
 (segment (start 142.1 94.5) (end 145.95 94.5) (width 0.5) (layer "B.Cu") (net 3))
 (segment (start 145.95 94.5) (end 146.5 95.05) (width 0.5) (layer "B.Cu") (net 3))
 (segment (start 156.6 95.05) (end 157.15 94.5) (width 0.5) (layer "B.Cu") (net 3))
 (segment (start 146.5 95.05) (end 156.6 95.05) (width 0.5) (layer "B.Cu") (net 3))
 (segment (start 146.519277 96.480723) (end 148.830723 96.480723) (width 0.2) (layer "F.Cu") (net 1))
 (segment (start 146.519277 95.855723) (end 146.519277 96.480723) (width 0.2) (layer "F.Cu") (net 1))
 (segment (start 146.5 97.175) (end 146.5 96.5) (width 0.2) (layer "F.Cu") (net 1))
 (segment (start 152.269277 96.480723) (end 152.9 95.85) (width 0.2) (layer "F.Cu") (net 1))
 (segment (start 149.55 96.480723) (end 149.55 97.2) (width 0.2) (layer "F.Cu") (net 1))
 (segment (start 152.9 97.15) (end 152.9 97.111446) (width 0.2) (layer "F.Cu") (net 1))
 (segment (start 149.55 95.8) (end 149.55 96.480723) (width 0.2) (layer "F.Cu") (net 1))
 (segment (start 146.5 96.5) (end 146.519277 96.480723) (width 0.2) (layer "F.Cu") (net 1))
 (segment (start 152.9 97.111446) (end 152.269277 96.480723) (width 0.2) (layer "F.Cu") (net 1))
 (segment (start 146.55 95.825) (end 146.519277 95.855723) (width 0.2) (layer "F.Cu") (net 1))
 (segment (start 149.55 97.2) (end 149.55 98.0735) (width 0.2) (layer "F.Cu") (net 1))
 (segment (start 149.55 96.480723) (end 152.269277 96.480723) (width 0.2) (layer "F.Cu") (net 1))
 (segment (start 148.830723 96.480723) (end 149.55 96.480723) (width 0.2) (layer "F.Cu") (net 1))
 (segment (start 152.9 95.85) (end 152.9 95.775) (width 0.2) (layer "F.Cu") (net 1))
 (via (at 149.55 98.0735) (size 0.5) (drill 0.2) (layers "F.Cu" "B.Cu") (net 1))
 (segment (start 149.5 98.5) (end 158.6 98.5) (width 0.5) (layer "B.Cu") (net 1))
 (segment (start 149.55 98.45) (end 149.5 98.5) (width 0.2) (layer "B.Cu") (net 1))
 (segment (start 149.55 98.0735) (end 149.55 98.45) (width 0.2) (layer "B.Cu") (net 1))
 (segment (start 142.4 98.5) (end 149.5 98.5) (width 0.5) (layer "B.Cu") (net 1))
 (segment (start 142.6 96.5) (end 158.65 96.5) (width 0.5) (layer "B.Cu") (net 19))
 (segment (start 142.3 100.5) (end 158.5 100.5) (width 0.5) (layer "B.Cu") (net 20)))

